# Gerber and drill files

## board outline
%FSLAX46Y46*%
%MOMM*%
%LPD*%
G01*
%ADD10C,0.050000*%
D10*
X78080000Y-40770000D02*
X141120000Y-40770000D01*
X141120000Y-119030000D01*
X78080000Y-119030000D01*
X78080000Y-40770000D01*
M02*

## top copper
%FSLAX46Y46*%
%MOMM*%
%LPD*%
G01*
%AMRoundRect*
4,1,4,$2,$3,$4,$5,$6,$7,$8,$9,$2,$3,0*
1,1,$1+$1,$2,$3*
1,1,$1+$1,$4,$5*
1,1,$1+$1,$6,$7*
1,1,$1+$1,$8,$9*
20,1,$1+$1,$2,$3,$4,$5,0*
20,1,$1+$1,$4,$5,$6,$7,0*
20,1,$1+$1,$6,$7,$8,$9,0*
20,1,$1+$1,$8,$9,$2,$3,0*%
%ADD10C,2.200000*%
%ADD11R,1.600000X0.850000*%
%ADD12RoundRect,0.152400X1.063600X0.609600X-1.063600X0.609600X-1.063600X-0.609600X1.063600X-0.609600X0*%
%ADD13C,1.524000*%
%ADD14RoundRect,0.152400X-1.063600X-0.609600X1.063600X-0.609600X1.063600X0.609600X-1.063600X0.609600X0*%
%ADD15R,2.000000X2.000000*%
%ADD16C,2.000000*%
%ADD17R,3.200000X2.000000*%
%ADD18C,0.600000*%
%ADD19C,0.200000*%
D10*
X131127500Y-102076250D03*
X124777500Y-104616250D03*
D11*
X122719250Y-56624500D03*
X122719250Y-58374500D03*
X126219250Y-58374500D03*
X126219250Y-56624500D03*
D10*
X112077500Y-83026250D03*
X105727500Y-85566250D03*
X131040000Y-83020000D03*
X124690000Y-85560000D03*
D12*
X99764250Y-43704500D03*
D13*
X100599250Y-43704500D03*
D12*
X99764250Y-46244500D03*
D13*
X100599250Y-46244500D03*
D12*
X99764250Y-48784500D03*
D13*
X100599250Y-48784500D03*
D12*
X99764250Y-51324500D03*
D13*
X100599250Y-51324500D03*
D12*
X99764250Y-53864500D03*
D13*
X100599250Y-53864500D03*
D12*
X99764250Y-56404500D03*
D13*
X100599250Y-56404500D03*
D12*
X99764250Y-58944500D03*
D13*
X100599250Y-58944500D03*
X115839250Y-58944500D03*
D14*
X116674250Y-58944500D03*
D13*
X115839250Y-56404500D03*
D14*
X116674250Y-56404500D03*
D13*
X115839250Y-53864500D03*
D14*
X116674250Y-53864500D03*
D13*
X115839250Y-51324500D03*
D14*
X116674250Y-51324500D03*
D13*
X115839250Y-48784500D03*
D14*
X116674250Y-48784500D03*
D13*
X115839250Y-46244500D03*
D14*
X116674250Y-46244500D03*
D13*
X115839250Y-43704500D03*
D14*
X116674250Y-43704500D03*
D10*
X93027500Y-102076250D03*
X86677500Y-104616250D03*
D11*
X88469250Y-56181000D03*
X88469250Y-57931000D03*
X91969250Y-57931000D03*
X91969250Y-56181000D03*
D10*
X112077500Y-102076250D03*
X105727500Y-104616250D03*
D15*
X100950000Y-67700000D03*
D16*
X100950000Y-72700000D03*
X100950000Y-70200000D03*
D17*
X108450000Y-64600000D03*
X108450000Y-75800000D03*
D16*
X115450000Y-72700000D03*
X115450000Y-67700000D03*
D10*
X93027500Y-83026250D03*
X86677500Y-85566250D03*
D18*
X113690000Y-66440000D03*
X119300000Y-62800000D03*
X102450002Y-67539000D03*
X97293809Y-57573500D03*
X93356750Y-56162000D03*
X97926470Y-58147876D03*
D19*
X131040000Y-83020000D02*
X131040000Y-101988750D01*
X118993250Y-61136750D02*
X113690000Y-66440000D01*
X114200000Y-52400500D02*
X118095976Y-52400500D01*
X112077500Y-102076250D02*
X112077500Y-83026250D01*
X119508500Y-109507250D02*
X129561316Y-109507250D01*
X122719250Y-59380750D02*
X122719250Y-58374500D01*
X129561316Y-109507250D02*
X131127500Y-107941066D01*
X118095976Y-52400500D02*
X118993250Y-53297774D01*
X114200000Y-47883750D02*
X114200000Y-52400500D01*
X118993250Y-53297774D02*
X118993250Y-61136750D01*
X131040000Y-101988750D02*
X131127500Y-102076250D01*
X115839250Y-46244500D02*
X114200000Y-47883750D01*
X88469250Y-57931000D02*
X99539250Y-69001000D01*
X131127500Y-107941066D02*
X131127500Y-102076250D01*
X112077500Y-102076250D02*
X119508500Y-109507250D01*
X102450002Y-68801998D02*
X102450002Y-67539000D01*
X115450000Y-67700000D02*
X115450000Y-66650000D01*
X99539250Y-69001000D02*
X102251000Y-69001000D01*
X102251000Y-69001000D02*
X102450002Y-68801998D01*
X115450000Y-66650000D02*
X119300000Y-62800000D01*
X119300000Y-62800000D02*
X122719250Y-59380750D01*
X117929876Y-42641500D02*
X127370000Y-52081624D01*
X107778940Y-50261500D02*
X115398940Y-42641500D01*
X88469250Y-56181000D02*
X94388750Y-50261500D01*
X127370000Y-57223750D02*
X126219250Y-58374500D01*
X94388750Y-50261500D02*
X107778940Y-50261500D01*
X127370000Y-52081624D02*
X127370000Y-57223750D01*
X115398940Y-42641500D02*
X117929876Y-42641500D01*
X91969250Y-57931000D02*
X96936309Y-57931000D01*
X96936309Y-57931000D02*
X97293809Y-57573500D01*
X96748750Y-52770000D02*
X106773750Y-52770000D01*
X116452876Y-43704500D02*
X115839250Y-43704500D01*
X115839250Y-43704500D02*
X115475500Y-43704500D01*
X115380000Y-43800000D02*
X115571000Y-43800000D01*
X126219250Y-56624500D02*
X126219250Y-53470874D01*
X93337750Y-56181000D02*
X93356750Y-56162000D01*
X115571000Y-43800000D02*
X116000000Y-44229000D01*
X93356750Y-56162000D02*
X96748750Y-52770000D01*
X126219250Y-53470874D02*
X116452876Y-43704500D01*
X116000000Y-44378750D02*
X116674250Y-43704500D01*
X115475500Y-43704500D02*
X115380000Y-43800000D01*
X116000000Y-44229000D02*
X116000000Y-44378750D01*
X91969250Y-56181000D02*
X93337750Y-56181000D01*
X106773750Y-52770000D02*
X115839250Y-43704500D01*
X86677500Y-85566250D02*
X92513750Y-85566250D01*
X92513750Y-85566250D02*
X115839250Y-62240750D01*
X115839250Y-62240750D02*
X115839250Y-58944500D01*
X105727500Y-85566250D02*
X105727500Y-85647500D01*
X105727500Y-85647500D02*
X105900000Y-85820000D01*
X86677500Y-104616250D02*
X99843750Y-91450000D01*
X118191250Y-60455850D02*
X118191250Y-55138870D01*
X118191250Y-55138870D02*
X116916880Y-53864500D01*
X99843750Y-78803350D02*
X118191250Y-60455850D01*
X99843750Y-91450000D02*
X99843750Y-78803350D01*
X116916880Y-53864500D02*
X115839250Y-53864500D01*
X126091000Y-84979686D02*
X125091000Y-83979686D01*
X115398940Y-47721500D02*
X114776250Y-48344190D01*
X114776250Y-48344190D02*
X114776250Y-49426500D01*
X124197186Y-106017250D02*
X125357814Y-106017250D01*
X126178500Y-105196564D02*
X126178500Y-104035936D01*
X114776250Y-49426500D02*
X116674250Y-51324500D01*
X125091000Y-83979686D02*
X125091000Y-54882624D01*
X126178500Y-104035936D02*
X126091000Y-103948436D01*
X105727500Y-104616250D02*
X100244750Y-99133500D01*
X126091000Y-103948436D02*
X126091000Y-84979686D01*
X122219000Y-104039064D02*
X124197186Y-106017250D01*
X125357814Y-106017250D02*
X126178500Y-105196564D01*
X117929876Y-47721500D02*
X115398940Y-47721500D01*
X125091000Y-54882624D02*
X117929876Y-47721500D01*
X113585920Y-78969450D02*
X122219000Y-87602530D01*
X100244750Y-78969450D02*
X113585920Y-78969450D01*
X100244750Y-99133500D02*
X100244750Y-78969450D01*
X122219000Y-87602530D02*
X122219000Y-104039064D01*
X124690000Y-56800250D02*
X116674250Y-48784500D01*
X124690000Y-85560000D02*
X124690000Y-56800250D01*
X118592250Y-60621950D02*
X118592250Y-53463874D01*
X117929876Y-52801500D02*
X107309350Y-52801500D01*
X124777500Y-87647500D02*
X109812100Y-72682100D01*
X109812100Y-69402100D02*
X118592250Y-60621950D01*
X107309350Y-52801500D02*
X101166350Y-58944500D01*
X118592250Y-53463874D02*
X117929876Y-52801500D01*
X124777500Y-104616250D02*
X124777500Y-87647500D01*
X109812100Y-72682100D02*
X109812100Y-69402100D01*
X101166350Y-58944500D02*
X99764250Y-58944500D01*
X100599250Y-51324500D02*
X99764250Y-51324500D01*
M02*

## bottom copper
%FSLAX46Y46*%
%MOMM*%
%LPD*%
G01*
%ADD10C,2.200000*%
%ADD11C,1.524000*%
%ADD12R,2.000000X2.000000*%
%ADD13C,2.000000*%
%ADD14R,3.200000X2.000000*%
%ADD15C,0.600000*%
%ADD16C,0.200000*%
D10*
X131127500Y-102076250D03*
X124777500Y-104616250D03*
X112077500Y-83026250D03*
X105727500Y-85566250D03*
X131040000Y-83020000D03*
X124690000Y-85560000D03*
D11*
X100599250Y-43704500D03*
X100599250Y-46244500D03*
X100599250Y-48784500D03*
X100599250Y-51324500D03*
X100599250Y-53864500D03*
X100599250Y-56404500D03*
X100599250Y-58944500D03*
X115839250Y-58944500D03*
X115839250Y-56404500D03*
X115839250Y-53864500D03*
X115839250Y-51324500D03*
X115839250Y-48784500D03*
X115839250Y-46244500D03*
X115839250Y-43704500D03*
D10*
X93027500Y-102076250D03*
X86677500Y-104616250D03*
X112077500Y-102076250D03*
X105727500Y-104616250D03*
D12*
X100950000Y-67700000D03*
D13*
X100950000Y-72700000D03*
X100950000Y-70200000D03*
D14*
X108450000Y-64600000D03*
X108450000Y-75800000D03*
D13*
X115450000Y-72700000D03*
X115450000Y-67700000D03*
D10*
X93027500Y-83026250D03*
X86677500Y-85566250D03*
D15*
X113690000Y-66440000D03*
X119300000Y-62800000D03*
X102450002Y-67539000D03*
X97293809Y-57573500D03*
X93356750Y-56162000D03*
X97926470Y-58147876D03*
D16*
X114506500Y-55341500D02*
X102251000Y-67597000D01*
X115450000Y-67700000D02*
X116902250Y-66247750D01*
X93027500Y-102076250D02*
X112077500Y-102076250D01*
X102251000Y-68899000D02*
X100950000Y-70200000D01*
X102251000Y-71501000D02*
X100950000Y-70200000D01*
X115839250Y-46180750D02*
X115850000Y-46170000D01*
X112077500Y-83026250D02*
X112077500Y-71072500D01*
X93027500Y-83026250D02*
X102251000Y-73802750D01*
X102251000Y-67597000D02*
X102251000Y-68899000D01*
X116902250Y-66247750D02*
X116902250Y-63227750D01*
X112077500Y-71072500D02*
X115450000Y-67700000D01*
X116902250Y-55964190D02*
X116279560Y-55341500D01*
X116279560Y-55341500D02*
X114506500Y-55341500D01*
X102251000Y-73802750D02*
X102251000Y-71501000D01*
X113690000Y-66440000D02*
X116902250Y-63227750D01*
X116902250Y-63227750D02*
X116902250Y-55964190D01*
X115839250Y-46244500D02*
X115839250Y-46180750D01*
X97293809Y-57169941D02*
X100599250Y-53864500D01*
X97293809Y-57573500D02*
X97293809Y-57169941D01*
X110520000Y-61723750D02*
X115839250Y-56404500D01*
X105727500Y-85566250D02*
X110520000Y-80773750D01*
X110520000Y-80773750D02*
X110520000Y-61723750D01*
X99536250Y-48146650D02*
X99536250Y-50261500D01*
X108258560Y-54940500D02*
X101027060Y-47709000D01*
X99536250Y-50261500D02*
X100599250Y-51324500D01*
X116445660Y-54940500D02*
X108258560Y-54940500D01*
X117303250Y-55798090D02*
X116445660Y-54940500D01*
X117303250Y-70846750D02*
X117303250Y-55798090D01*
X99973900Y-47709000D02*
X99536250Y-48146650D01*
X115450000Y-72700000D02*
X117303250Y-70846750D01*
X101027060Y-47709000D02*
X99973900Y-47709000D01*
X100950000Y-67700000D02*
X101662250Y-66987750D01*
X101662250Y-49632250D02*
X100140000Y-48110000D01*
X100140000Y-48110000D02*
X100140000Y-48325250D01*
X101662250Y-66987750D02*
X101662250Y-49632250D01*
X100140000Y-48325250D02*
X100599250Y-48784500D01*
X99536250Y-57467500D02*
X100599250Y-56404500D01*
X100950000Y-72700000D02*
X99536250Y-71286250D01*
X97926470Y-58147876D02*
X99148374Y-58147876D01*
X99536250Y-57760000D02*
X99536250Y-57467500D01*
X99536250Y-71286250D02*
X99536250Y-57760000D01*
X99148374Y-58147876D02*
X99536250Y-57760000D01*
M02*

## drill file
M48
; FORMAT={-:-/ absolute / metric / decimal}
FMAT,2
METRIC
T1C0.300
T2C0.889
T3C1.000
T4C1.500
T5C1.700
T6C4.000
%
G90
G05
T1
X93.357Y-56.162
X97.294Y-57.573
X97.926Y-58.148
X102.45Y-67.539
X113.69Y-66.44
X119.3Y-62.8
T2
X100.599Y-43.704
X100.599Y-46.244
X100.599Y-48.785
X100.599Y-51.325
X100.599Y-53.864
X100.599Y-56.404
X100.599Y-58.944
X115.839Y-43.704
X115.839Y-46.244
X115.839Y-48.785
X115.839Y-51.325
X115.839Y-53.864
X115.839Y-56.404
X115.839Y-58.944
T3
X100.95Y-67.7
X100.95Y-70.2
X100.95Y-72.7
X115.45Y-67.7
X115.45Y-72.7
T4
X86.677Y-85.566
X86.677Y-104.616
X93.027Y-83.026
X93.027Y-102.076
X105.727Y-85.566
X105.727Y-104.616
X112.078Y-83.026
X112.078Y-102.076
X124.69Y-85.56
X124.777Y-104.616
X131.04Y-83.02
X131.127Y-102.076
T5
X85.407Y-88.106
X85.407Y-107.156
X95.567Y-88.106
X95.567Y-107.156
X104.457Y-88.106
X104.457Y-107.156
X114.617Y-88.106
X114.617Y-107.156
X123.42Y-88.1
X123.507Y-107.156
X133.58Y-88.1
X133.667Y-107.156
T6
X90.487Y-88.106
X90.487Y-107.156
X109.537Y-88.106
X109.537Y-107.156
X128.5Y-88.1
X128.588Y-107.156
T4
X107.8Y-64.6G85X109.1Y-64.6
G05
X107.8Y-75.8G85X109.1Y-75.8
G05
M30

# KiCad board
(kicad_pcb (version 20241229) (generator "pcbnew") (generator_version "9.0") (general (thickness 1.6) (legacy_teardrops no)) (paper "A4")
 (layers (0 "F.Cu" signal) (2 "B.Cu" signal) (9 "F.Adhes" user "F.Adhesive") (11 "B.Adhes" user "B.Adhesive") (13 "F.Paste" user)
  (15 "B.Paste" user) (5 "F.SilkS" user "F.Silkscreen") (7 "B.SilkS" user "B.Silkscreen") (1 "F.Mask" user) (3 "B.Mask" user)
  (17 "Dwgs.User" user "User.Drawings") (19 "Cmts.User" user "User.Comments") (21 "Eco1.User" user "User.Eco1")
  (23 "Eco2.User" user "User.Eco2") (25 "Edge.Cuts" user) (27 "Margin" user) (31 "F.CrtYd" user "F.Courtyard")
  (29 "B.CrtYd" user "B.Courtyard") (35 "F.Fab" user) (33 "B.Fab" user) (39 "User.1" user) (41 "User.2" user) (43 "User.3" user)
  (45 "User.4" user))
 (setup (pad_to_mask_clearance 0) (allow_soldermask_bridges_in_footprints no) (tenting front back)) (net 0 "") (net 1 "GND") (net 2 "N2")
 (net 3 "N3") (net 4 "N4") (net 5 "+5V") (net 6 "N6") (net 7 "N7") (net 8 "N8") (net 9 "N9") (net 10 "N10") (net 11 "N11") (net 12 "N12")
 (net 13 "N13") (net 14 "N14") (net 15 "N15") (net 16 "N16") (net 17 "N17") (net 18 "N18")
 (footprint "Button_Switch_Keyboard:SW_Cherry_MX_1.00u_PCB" (layer "F.Cu") (at 131.1275 102.07625)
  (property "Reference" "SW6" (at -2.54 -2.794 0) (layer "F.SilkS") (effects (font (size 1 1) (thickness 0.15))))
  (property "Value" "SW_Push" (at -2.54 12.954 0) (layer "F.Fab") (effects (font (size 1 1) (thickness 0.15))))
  (pad "" np_thru_hole circle (at -7.62 5.08) (size 1.7 1.7) (drill 1.7) (layers "*.Cu" "*.Mask"))
  (pad "" np_thru_hole circle (at -2.54 5.08) (size 4 4) (drill 4) (layers "*.Cu" "*.Mask"))
  (pad "" np_thru_hole circle (at 2.54 5.08) (size 1.7 1.7) (drill 1.7) (layers "*.Cu" "*.Mask"))
  (pad "1" thru_hole circle (at 0 0) (size 2.2 2.2) (drill 1.5) (layers "*.Cu" "*.Mask") (remove_unused_layers no) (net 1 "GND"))
  (pad "2" thru_hole circle (at -6.35 2.54) (size 2.2 2.2) (drill 1.5) (layers "*.Cu" "*.Mask") (remove_unused_layers no) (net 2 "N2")))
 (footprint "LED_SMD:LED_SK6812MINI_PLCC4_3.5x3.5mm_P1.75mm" (layer "F.Cu") (at 124.46925 57.4995)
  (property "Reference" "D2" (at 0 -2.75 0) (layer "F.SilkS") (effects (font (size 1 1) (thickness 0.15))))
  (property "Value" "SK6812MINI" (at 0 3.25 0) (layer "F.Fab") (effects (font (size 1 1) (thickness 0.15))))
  (pad "1" smd rect (at -1.75 -0.875) (size 1.6 0.85) (layers "F.Cu" "F.Mask" "F.Paste") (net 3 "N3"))
  (pad "2" smd rect (at -1.75 0.875) (size 1.6 0.85) (layers "F.Cu" "F.Mask" "F.Paste") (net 1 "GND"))
  (pad "3" smd rect (at 1.75 0.875) (size 1.6 0.85) (layers "F.Cu" "F.Mask" "F.Paste") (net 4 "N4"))
  (pad "4" smd rect (at 1.75 -0.875) (size 1.6 0.85) (layers "F.Cu" "F.Mask" "F.Paste") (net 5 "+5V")))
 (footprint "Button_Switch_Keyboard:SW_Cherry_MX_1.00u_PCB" (layer "F.Cu") (at 112.0775 83.02625)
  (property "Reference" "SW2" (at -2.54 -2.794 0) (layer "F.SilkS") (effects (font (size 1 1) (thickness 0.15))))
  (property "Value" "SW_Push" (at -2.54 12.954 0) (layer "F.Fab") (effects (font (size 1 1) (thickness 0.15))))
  (pad "" np_thru_hole circle (at -7.62 5.08) (size 1.7 1.7) (drill 1.7) (layers "*.Cu" "*.Mask"))
  (pad "" np_thru_hole circle (at -2.54 5.08) (size 4 4) (drill 4) (layers "*.Cu" "*.Mask"))
  (pad "" np_thru_hole circle (at 2.54 5.08) (size 1.7 1.7) (drill 1.7) (layers "*.Cu" "*.Mask"))
  (pad "1" thru_hole circle (at 0 0) (size 2.2 2.2) (drill 1.5) (layers "*.Cu" "*.Mask") (remove_unused_layers no) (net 1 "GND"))
  (pad "2" thru_hole circle (at -6.35 2.54) (size 2.2 2.2) (drill 1.5) (layers "*.Cu" "*.Mask") (remove_unused_layers no) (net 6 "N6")))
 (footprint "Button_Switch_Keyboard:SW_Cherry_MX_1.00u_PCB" (layer "F.Cu") (at 131.04 83.02)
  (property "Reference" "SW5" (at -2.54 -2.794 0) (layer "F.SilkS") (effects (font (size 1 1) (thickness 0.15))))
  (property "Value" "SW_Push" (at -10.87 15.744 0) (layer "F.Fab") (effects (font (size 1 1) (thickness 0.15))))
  (pad "" np_thru_hole circle (at -7.62 5.08) (size 1.7 1.7) (drill 1.7) (layers "*.Cu" "*.Mask"))
  (pad "" np_thru_hole circle (at -2.54 5.08) (size 4 4) (drill 4) (layers "*.Cu" "*.Mask"))
  (pad "" np_thru_hole circle (at 2.54 5.08) (size 1.7 1.7) (drill 1.7) (layers "*.Cu" "*.Mask"))
  (pad "1" thru_hole circle (at 0 0) (size 2.2 2.2) (drill 1.5) (layers "*.Cu" "*.Mask") (remove_unused_layers no) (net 1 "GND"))
  (pad "2" thru_hole circle (at -6.35 2.54) (size 2.2 2.2) (drill 1.5) (layers "*.Cu" "*.Mask") (remove_unused_layers no) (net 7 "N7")))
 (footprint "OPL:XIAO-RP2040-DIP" (layer "F.Cu") (at 108.21925 51.3245)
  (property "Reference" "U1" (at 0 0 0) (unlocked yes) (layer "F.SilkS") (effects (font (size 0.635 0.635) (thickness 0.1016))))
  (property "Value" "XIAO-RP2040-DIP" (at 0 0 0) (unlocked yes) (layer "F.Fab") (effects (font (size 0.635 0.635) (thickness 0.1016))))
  (pad "1" smd roundrect (at -8.455 -7.62 180) (size 2.432 1.524) (layers "F.Cu" "F.Mask") (roundrect_rratio 0.1) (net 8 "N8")
   (thermal_bridge_angle 45))
  (pad "1" thru_hole circle (at -7.62 -7.62 180) (size 1.524 1.524) (drill 0.889) (layers "*.Cu" "*.Mask") (remove_unused_layers no)
   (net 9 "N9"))
  (pad "2" smd roundrect (at -8.455 -5.08 180) (size 2.432 1.524) (layers "F.Cu" "F.Mask") (roundrect_rratio 0.1) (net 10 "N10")
   (thermal_bridge_angle 45))
  (pad "2" thru_hole circle (at -7.62 -5.08 180) (size 1.524 1.524) (drill 0.889) (layers "*.Cu" "*.Mask") (remove_unused_layers no)
   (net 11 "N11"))
  (pad "3" smd roundrect (at -8.455 -2.54 180) (size 2.432 1.524) (layers "F.Cu" "F.Mask") (roundrect_rratio 0.1) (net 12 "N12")
   (thermal_bridge_angle 45))
  (pad "3" thru_hole circle (at -7.62 -2.54 180) (size 1.524 1.524) (drill 0.889) (layers "*.Cu" "*.Mask") (remove_unused_layers no)
   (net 12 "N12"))
  (pad "4" smd roundrect (at -8.455 0 180) (size 2.432 1.524) (layers "F.Cu" "F.Mask") (roundrect_rratio 0.1) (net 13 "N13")
   (thermal_bridge_angle 45))
  (pad "4" thru_hole circle (at -7.62 0 180) (size 1.524 1.524) (drill 0.889) (layers "*.Cu" "*.Mask") (remove_unused_layers no)
   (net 13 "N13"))
  (pad "5" smd roundrect (at -8.455 2.54 180) (size 2.432 1.524) (layers "F.Cu" "F.Mask") (roundrect_rratio 0.1) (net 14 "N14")
   (thermal_bridge_angle 45))
  (pad "5" thru_hole circle (at -7.62 2.54 180) (size 1.524 1.524) (drill 0.889) (layers "*.Cu" "*.Mask") (remove_unused_layers no)
   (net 14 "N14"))
  (pad "6" smd roundrect (at -8.455 5.08 180) (size 2.432 1.524) (layers "F.Cu" "F.Mask") (roundrect_rratio 0.1) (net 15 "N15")
   (thermal_bridge_angle 45))
  (pad "6" thru_hole circle (at -7.62 5.08 180) (size 1.524 1.524) (drill 0.889) (layers "*.Cu" "*.Mask") (remove_unused_layers no)
   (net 15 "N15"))
  (pad "7" smd roundrect (at -8.455 7.62 180) (size 2.432 1.524) (layers "F.Cu" "F.Mask") (roundrect_rratio 0.1) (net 2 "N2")
   (thermal_bridge_angle 45))
  (pad "7" thru_hole circle (at -7.62 7.62 180) (size 1.524 1.524) (drill 0.889) (layers "*.Cu" "*.Mask") (remove_unused_layers no)
   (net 2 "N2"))
  (pad "8" thru_hole circle (at 7.62 7.62) (size 1.524 1.524) (drill 0.889) (layers "*.Cu" "*.Mask") (remove_unused_layers no)
   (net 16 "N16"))
  (pad "8" smd roundrect (at 8.455 7.62) (size 2.432 1.524) (layers "F.Cu" "F.Mask") (roundrect_rratio 0.1) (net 16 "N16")
   (thermal_bridge_angle 45))
  (pad "9" thru_hole circle (at 7.62 5.08) (size 1.524 1.524) (drill 0.889) (layers "*.Cu" "*.Mask") (remove_unused_layers no) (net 6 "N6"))
  (pad "9" smd roundrect (at 8.455 5.08) (size 2.432 1.524) (layers "F.Cu" "F.Mask") (roundrect_rratio 0.1) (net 6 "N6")
   (thermal_bridge_angle 45))
  (pad "10" thru_hole circle (at 7.62 2.54) (size 1.524 1.524) (drill 0.889) (layers "*.Cu" "*.Mask") (remove_unused_layers no)
   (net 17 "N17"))
  (pad "10" smd roundrect (at 8.455 2.54) (size 2.432 1.524) (layers "F.Cu" "F.Mask") (roundrect_rratio 0.1) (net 17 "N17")
   (thermal_bridge_angle 45))
  (pad "11" thru_hole circle (at 7.62 0) (size 1.524 1.524) (drill 0.889) (layers "*.Cu" "*.Mask") (remove_unused_layers no) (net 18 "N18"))
  (pad "11" smd roundrect (at 8.455 0) (size 2.432 1.524) (layers "F.Cu" "F.Mask") (roundrect_rratio 0.1) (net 18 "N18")
   (thermal_bridge_angle 45))
  (pad "12" thru_hole circle (at 7.62 -2.54) (size 1.524 1.524) (drill 0.889) (layers "*.Cu" "*.Mask") (remove_unused_layers no)
   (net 7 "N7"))
  (pad "12" smd roundrect (at 8.455 -2.54) (size 2.432 1.524) (layers "F.Cu" "F.Mask") (roundrect_rratio 0.1) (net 7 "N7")
   (thermal_bridge_angle 45))
  (pad "13" thru_hole circle (at 7.62 -5.08) (size 1.524 1.524) (drill 0.889) (layers "*.Cu" "*.Mask") (remove_unused_layers no)
   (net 1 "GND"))
  (pad "13" smd roundrect (at 8.455 -5.08) (size 2.432 1.524) (layers "F.Cu" "F.Mask") (roundrect_rratio 0.1) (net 1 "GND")
   (thermal_bridge_angle 45))
  (pad "14" thru_hole circle (at 7.62 -7.62) (size 1.524 1.524) (drill 0.889) (layers "*.Cu" "*.Mask") (remove_unused_layers no)
   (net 5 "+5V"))
  (pad "14" smd roundrect (at 8.455 -7.62) (size 2.432 1.524) (layers "F.Cu" "F.Mask") (roundrect_rratio 0.1) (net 5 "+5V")
   (thermal_bridge_angle 45)))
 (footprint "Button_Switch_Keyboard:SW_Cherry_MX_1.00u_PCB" (layer "F.Cu") (at 93.0275 102.07625)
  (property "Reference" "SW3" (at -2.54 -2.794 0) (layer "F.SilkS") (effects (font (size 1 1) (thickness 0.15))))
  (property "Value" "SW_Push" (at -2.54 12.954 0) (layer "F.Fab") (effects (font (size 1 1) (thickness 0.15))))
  (pad "" np_thru_hole circle (at -7.62 5.08) (size 1.7 1.7) (drill 1.7) (layers "*.Cu" "*.Mask"))
  (pad "" np_thru_hole circle (at -2.54 5.08) (size 4 4) (drill 4) (layers "*.Cu" "*.Mask"))
  (pad "" np_thru_hole circle (at 2.54 5.08) (size 1.7 1.7) (drill 1.7) (layers "*.Cu" "*.Mask"))
  (pad "1" thru_hole circle (at 0 0) (size 2.2 2.2) (drill 1.5) (layers "*.Cu" "*.Mask") (remove_unused_layers no) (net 1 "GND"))
  (pad "2" thru_hole circle (at -6.35 2.54) (size 2.2 2.2) (drill 1.5) (layers "*.Cu" "*.Mask") (remove_unused_layers no) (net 17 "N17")))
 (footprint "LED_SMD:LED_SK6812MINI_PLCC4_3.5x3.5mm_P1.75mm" (layer "F.Cu") (at 90.21925 57.056)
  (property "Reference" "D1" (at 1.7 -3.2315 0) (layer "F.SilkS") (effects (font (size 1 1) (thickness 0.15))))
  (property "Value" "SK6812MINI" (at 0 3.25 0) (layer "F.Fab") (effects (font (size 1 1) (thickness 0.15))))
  (pad "1" smd rect (at -1.75 -0.875) (size 1.6 0.85) (layers "F.Cu" "F.Mask" "F.Paste") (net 4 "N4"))
  (pad "2" smd rect (at -1.75 0.875) (size 1.6 0.85) (layers "F.Cu" "F.Mask" "F.Paste") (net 1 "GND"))
  (pad "3" smd rect (at 1.75 0.875) (size 1.6 0.85) (layers "F.Cu" "F.Mask" "F.Paste") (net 14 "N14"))
  (pad "4" smd rect (at 1.75 -0.875) (size 1.6 0.85) (layers "F.Cu" "F.Mask" "F.Paste") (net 5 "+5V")))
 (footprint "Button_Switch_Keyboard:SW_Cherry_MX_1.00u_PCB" (layer "F.Cu") (at 112.0775 102.07625)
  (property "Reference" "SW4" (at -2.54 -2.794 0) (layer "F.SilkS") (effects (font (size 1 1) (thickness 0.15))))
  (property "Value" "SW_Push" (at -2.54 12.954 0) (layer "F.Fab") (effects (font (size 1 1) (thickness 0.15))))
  (pad "" np_thru_hole circle (at -7.62 5.08) (size 1.7 1.7) (drill 1.7) (layers "*.Cu" "*.Mask"))
  (pad "" np_thru_hole circle (at -2.54 5.08) (size 4 4) (drill 4) (layers "*.Cu" "*.Mask"))
  (pad "" np_thru_hole circle (at 2.54 5.08) (size 1.7 1.7) (drill 1.7) (layers "*.Cu" "*.Mask"))
  (pad "1" thru_hole circle (at 0 0) (size 2.2 2.2) (drill 1.5) (layers "*.Cu" "*.Mask") (remove_unused_layers no) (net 1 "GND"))
  (pad "2" thru_hole circle (at -6.35 2.54) (size 2.2 2.2) (drill 1.5) (layers "*.Cu" "*.Mask") (remove_unused_layers no) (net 18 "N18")))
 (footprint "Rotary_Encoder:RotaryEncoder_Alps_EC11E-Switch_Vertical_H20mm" (layer "F.Cu") (at 100.95 67.7)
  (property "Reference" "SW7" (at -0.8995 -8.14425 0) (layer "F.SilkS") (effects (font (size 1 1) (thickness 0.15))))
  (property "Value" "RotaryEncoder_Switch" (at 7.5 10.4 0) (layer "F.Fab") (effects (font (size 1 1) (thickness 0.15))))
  (pad "A" thru_hole rect (at 0 0) (size 2 2) (drill 1) (layers "*.Cu" "*.Mask") (remove_unused_layers no) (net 12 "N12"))
  (pad "B" thru_hole circle (at 0 5) (size 2 2) (drill 1) (layers "*.Cu" "*.Mask") (remove_unused_layers no) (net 15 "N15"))
  (pad "C" thru_hole circle (at 0 2.5) (size 2 2) (drill 1) (layers "*.Cu" "*.Mask") (remove_unused_layers no) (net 1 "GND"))
  (pad "MP" thru_hole rect (at 7.5 -3.1) (size 3.2 2) (drill oval 2.8 1.5) (layers "*.Cu" "*.Mask") (remove_unused_layers no))
  (pad "MP" thru_hole rect (at 7.5 8.1) (size 3.2 2) (drill oval 2.8 1.5) (layers "*.Cu" "*.Mask") (remove_unused_layers no))
  (pad "S1" thru_hole circle (at 14.5 5) (size 2 2) (drill 1) (layers "*.Cu" "*.Mask") (remove_unused_layers no) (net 13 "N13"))
  (pad "S2" thru_hole circle (at 14.5 0) (size 2 2) (drill 1) (layers "*.Cu" "*.Mask") (remove_unused_layers no) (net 1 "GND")))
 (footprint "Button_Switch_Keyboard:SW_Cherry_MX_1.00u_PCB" (layer "F.Cu") (at 93.0275 83.02625)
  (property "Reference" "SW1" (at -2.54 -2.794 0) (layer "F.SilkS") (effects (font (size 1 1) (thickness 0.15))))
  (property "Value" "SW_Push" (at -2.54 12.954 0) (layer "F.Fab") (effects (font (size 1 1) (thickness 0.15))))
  (pad "" np_thru_hole circle (at -7.62 5.08) (size 1.7 1.7) (drill 1.7) (layers "*.Cu" "*.Mask"))
  (pad "" np_thru_hole circle (at -2.54 5.08) (size 4 4) (drill 4) (layers "*.Cu" "*.Mask"))
  (pad "" np_thru_hole circle (at 2.54 5.08) (size 1.7 1.7) (drill 1.7) (layers "*.Cu" "*.Mask"))
  (pad "1" thru_hole circle (at 0 0) (size 2.2 2.2) (drill 1.5) (layers "*.Cu" "*.Mask") (remove_unused_layers no) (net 1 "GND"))
  (pad "2" thru_hole circle (at -6.35 2.54) (size 2.2 2.2) (drill 1.5) (layers "*.Cu" "*.Mask") (remove_unused_layers no) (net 16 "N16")))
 (gr_rect (start 78.08 40.77) (end 141.12 119.03) (stroke (width 0.05) (type default)) (fill no) (layer "Edge.Cuts"))
 (segment (start 131.04 83.02) (end 131.04 101.98875) (width 0.2) (layer "F.Cu") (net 1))
 (segment (start 118.99325 61.13675) (end 113.69 66.44) (width 0.2) (layer "F.Cu") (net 1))
 (segment (start 114.2 52.4005) (end 118.095976 52.4005) (width 0.2) (layer "F.Cu") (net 1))
 (segment (start 112.0775 102.07625) (end 112.0775 83.02625) (width 0.2) (layer "F.Cu") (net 1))
 (segment (start 119.5085 109.50725) (end 129.561316 109.50725) (width 0.2) (layer "F.Cu") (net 1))
 (segment (start 122.71925 59.38075) (end 122.71925 58.3745) (width 0.2) (layer "F.Cu") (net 1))
 (segment (start 129.561316 109.50725) (end 131.1275 107.941066) (width 0.2) (layer "F.Cu") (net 1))
 (segment (start 118.095976 52.4005) (end 118.99325 53.297774) (width 0.2) (layer "F.Cu") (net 1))
 (segment (start 114.2 47.88375) (end 114.2 52.4005) (width 0.2) (layer "F.Cu") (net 1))
 (segment (start 118.99325 53.297774) (end 118.99325 61.13675) (width 0.2) (layer "F.Cu") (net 1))
 (segment (start 131.04 101.98875) (end 131.1275 102.07625) (width 0.2) (layer "F.Cu") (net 1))
 (segment (start 115.83925 46.2445) (end 114.2 47.88375) (width 0.2) (layer "F.Cu") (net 1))
 (segment (start 88.46925 57.931) (end 99.53925 69.001) (width 0.2) (layer "F.Cu") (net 1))
 (segment (start 131.1275 107.941066) (end 131.1275 102.07625) (width 0.2) (layer "F.Cu") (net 1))
 (segment (start 112.0775 102.07625) (end 119.5085 109.50725) (width 0.2) (layer "F.Cu") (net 1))
 (segment (start 102.450002 68.801998) (end 102.450002 67.539) (width 0.2) (layer "F.Cu") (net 1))
 (segment (start 115.45 67.7) (end 115.45 66.65) (width 0.2) (layer "F.Cu") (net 1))
 (segment (start 99.53925 69.001) (end 102.251 69.001) (width 0.2) (layer "F.Cu") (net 1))
 (segment (start 102.251 69.001) (end 102.450002 68.801998) (width 0.2) (layer "F.Cu") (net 1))
 (segment (start 115.45 66.65) (end 119.3 62.8) (width 0.2) (layer "F.Cu") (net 1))
 (segment (start 119.3 62.8) (end 122.71925 59.38075) (width 0.2) (layer "F.Cu") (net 1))
 (via (at 113.69 66.44) (size 0.6) (drill 0.3) (layers "F.Cu" "B.Cu") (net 1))
 (via (at 119.3 62.8) (size 0.6) (drill 0.3) (layers "F.Cu" "B.Cu") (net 1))
 (via (at 102.450002 67.539) (size 0.6) (drill 0.3) (layers "F.Cu" "B.Cu") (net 1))
 (segment (start 114.5065 55.3415) (end 102.251 67.597) (width 0.2) (layer "B.Cu") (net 1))
 (segment (start 115.45 67.7) (end 116.90225 66.24775) (width 0.2) (layer "B.Cu") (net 1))
 (segment (start 93.0275 102.07625) (end 112.0775 102.07625) (width 0.2) (layer "B.Cu") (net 1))
 (segment (start 102.251 68.899) (end 100.95 70.2) (width 0.2) (layer "B.Cu") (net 1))
 (segment (start 102.251 71.501) (end 100.95 70.2) (width 0.2) (layer "B.Cu") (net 1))
 (segment (start 115.83925 46.18075) (end 115.85 46.17) (width 0.2) (layer "B.Cu") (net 1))
 (segment (start 112.0775 83.02625) (end 112.0775 71.0725) (width 0.2) (layer "B.Cu") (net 1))
 (segment (start 93.0275 83.02625) (end 102.251 73.80275) (width 0.2) (layer "B.Cu") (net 1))
 (segment (start 102.251 67.597) (end 102.251 68.899) (width 0.2) (layer "B.Cu") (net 1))
 (segment (start 116.90225 66.24775) (end 116.90225 63.22775) (width 0.2) (layer "B.Cu") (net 1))
 (segment (start 112.0775 71.0725) (end 115.45 67.7) (width 0.2) (layer "B.Cu") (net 1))
 (segment (start 116.90225 55.96419) (end 116.27956 55.3415) (width 0.2) (layer "B.Cu") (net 1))
 (segment (start 116.27956 55.3415) (end 114.5065 55.3415) (width 0.2) (layer "B.Cu") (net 1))
 (segment (start 102.251 73.80275) (end 102.251 71.501) (width 0.2) (layer "B.Cu") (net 1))
 (segment (start 113.69 66.44) (end 116.90225 63.22775) (width 0.2) (layer "B.Cu") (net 1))
 (segment (start 116.90225 63.22775) (end 116.90225 55.96419) (width 0.2) (layer "B.Cu") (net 1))
 (segment (start 115.83925 46.2445) (end 115.83925 46.18075) (width 0.2) (layer "B.Cu") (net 1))
 (segment (start 117.929876 42.6415) (end 127.37 52.081624) (width 0.2) (layer "F.Cu") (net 4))
 (segment (start 107.77894 50.2615) (end 115.39894 42.6415) (width 0.2) (layer "F.Cu") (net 4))
 (segment (start 88.46925 56.181) (end 94.38875 50.2615) (width 0.2) (layer "F.Cu") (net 4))
 (segment (start 127.37 57.22375) (end 126.21925 58.3745) (width 0.2) (layer "F.Cu") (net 4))
 (segment (start 94.38875 50.2615) (end 107.77894 50.2615) (width 0.2) (layer "F.Cu") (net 4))
 (segment (start 127.37 52.081624) (end 127.37 57.22375) (width 0.2) (layer "F.Cu") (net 4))
 (segment (start 115.39894 42.6415) (end 117.929876 42.6415) (width 0.2) (layer "F.Cu") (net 4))
 (segment (start 91.96925 57.931) (end 96.936309 57.931) (width 0.2) (layer "F.Cu") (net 14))
 (segment (start 96.936309 57.931) (end 97.293809 57.5735) (width 0.2) (layer "F.Cu") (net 14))
 (via (at 97.293809 57.5735) (size 0.6) (drill 0.3) (layers "F.Cu" "B.Cu") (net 14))
 (segment (start 97.293809 57.169941) (end 100.59925 53.8645) (width 0.2) (layer "B.Cu") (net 14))
 (segment (start 97.293809 57.5735) (end 97.293809 57.169941) (width 0.2) (layer "B.Cu") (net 14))
 (segment (start 96.74875 52.77) (end 106.77375 52.77) (width 0.2) (layer "F.Cu") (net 5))
 (segment (start 116.452876 43.7045) (end 115.83925 43.7045) (width 0.2) (layer "F.Cu") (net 5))
 (segment (start 115.83925 43.7045) (end 115.4755 43.7045) (width 0.2) (layer "F.Cu") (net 5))
 (segment (start 115.38 43.8) (end 115.571 43.8) (width 0.2) (layer "F.Cu") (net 5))
 (segment (start 126.21925 56.6245) (end 126.21925 53.470874) (width 0.2) (layer "F.Cu") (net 5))
 (segment (start 93.33775 56.181) (end 93.35675 56.162) (width 0.2) (layer "F.Cu") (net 5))
 (segment (start 115.571 43.8) (end 116 44.229) (width 0.2) (layer "F.Cu") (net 5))
 (segment (start 93.35675 56.162) (end 96.74875 52.77) (width 0.2) (layer "F.Cu") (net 5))
 (segment (start 126.21925 53.470874) (end 116.452876 43.7045) (width 0.2) (layer "F.Cu") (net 5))
 (segment (start 116 44.37875) (end 116.67425 43.7045) (width 0.2) (layer "F.Cu") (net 5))
 (segment (start 115.4755 43.7045) (end 115.38 43.8) (width 0.2) (layer "F.Cu") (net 5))
 (segment (start 116 44.229) (end 116 44.37875) (width 0.2) (layer "F.Cu") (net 5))
 (segment (start 91.96925 56.181) (end 93.33775 56.181) (width 0.2) (layer "F.Cu") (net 5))
 (segment (start 106.77375 52.77) (end 115.83925 43.7045) (width 0.2) (layer "F.Cu") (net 5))
 (via (at 93.35675 56.162) (size 0.6) (drill 0.3) (layers "F.Cu" "B.Cu") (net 5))
 (segment (start 86.6775 85.56625) (end 92.51375 85.56625) (width 0.2) (layer "F.Cu") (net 16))
 (segment (start 92.51375 85.56625) (end 115.83925 62.24075) (width 0.2) (layer "F.Cu") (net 16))
 (segment (start 115.83925 62.24075) (end 115.83925 58.9445) (width 0.2) (layer "F.Cu") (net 16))
 (segment (start 105.7275 85.56625) (end 105.7275 85.6475) (width 0.2) (layer "F.Cu") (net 6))
 (segment (start 105.7275 85.6475) (end 105.9 85.82) (width 0.2) (layer "F.Cu") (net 6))
 (segment (start 110.52 61.72375) (end 115.83925 56.4045) (width 0.2) (layer "B.Cu") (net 6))
 (segment (start 105.7275 85.56625) (end 110.52 80.77375) (width 0.2) (layer "B.Cu") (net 6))
 (segment (start 110.52 80.77375) (end 110.52 61.72375) (width 0.2) (layer "B.Cu") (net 6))
 (segment (start 86.6775 104.61625) (end 99.84375 91.45) (width 0.2) (layer "F.Cu") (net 17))
 (segment (start 118.19125 60.45585) (end 118.19125 55.13887) (width 0.2) (layer "F.Cu") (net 17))
 (segment (start 118.19125 55.13887) (end 116.91688 53.8645) (width 0.2) (layer "F.Cu") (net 17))
 (segment (start 99.84375 78.80335) (end 118.19125 60.45585) (width 0.2) (layer "F.Cu") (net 17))
 (segment (start 99.84375 91.45) (end 99.84375 78.80335) (width 0.2) (layer "F.Cu") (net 17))
 (segment (start 116.91688 53.8645) (end 115.83925 53.8645) (width 0.2) (layer "F.Cu") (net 17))
 (segment (start 126.091 84.979686) (end 125.091 83.979686) (width 0.2) (layer "F.Cu") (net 18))
 (segment (start 115.39894 47.7215) (end 114.77625 48.34419) (width 0.2) (layer "F.Cu") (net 18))
 (segment (start 114.77625 48.34419) (end 114.77625 49.4265) (width 0.2) (layer "F.Cu") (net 18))
 (segment (start 124.197186 106.01725) (end 125.357814 106.01725) (width 0.2) (layer "F.Cu") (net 18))
 (segment (start 126.1785 105.196564) (end 126.1785 104.035936) (width 0.2) (layer "F.Cu") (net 18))
 (segment (start 114.77625 49.4265) (end 116.67425 51.3245) (width 0.2) (layer "F.Cu") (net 18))
 (segment (start 125.091 83.979686) (end 125.091 54.882624) (width 0.2) (layer "F.Cu") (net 18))
 (segment (start 126.1785 104.035936) (end 126.091 103.948436) (width 0.2) (layer "F.Cu") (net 18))
 (segment (start 105.7275 104.61625) (end 100.24475 99.1335) (width 0.2) (layer "F.Cu") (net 18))
 (segment (start 126.091 103.948436) (end 126.091 84.979686) (width 0.2) (layer "F.Cu") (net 18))
 (segment (start 122.219 104.039064) (end 124.197186 106.01725) (width 0.2) (layer "F.Cu") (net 18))
 (segment (start 125.357814 106.01725) (end 126.1785 105.196564) (width 0.2) (layer "F.Cu") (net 18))
 (segment (start 117.929876 47.7215) (end 115.39894 47.7215) (width 0.2) (layer "F.Cu") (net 18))
 (segment (start 125.091 54.882624) (end 117.929876 47.7215) (width 0.2) (layer "F.Cu") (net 18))
 (segment (start 113.58592 78.96945) (end 122.219 87.60253) (width 0.2) (layer "F.Cu") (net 18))
 (segment (start 100.24475 78.96945) (end 113.58592 78.96945) (width 0.2) (layer "F.Cu") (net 18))
 (segment (start 100.24475 99.1335) (end 100.24475 78.96945) (width 0.2) (layer "F.Cu") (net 18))
 (segment (start 122.219 87.60253) (end 122.219 104.039064) (width 0.2) (layer "F.Cu") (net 18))
 (segment (start 124.69 56.80025) (end 116.67425 48.7845) (width 0.2) (layer "F.Cu") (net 7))
 (segment (start 124.69 85.56) (end 124.69 56.80025) (width 0.2) (layer "F.Cu") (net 7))
 (segment (start 118.59225 60.62195) (end 118.59225 53.463874) (width 0.2) (layer "F.Cu") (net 2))
 (segment (start 117.929876 52.8015) (end 107.30935 52.8015) (width 0.2) (layer "F.Cu") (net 2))
 (segment (start 124.7775 87.6475) (end 109.8121 72.6821) (width 0.2) (layer "F.Cu") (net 2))
 (segment (start 109.8121 69.4021) (end 118.59225 60.62195) (width 0.2) (layer "F.Cu") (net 2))
 (segment (start 107.30935 52.8015) (end 101.16635 58.9445) (width 0.2) (layer "F.Cu") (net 2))
 (segment (start 118.59225 53.463874) (end 117.929876 52.8015) (width 0.2) (layer "F.Cu") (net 2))
 (segment (start 124.7775 104.61625) (end 124.7775 87.6475) (width 0.2) (layer "F.Cu") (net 2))
 (segment (start 109.8121 72.6821) (end 109.8121 69.4021) (width 0.2) (layer "F.Cu") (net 2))
 (segment (start 101.16635 58.9445) (end 99.76425 58.9445) (width 0.2) (layer "F.Cu") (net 2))
 (segment (start 100.59925 51.3245) (end 99.76425 51.3245) (width 0.2) (layer "F.Cu") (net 13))
 (segment (start 99.53625 48.14665) (end 99.53625 50.2615) (width 0.2) (layer "B.Cu") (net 13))
 (segment (start 108.25856 54.9405) (end 101.02706 47.709) (width 0.2) (layer "B.Cu") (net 13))
 (segment (start 99.53625 50.2615) (end 100.59925 51.3245) (width 0.2) (layer "B.Cu") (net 13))
 (segment (start 116.44566 54.9405) (end 108.25856 54.9405) (width 0.2) (layer "B.Cu") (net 13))
 (segment (start 117.30325 55.79809) (end 116.44566 54.9405) (width 0.2) (layer "B.Cu") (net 13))
 (segment (start 117.30325 70.84675) (end 117.30325 55.79809) (width 0.2) (layer "B.Cu") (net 13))
 (segment (start 99.9739 47.709) (end 99.53625 48.14665) (width 0.2) (layer "B.Cu") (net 13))
 (segment (start 115.45 72.7) (end 117.30325 70.84675) (width 0.2) (layer "B.Cu") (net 13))
 (segment (start 101.02706 47.709) (end 99.9739 47.709) (width 0.2) (layer "B.Cu") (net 13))
 (segment (start 100.95 67.7) (end 101.66225 66.98775) (width 0.2) (layer "B.Cu") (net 12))
 (segment (start 101.66225 49.63225) (end 100.14 48.11) (width 0.2) (layer "B.Cu") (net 12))
 (segment (start 100.14 48.11) (end 100.14 48.32525) (width 0.2) (layer "B.Cu") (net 12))
 (segment (start 101.66225 66.98775) (end 101.66225 49.63225) (width 0.2) (layer "B.Cu") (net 12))
 (segment (start 100.14 48.32525) (end 100.59925 48.7845) (width 0.2) (layer "B.Cu") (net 12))
 (via (at 97.92647 58.147876) (size 0.6) (drill 0.3) (layers "F.Cu" "B.Cu") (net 15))
 (segment (start 99.53625 57.4675) (end 100.59925 56.4045) (width 0.2) (layer "B.Cu") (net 15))
 (segment (start 100.95 72.7) (end 99.53625 71.28625) (width 0.2) (layer "B.Cu") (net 15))
 (segment (start 97.92647 58.147876) (end 99.148374 58.147876) (width 0.2) (layer "B.Cu") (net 15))
 (segment (start 99.53625 57.76) (end 99.53625 57.4675) (width 0.2) (layer "B.Cu") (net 15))
 (segment (start 99.53625 71.28625) (end 99.53625 57.76) (width 0.2) (layer "B.Cu") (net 15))
 (segment (start 99.148374 58.147876) (end 99.53625 57.76) (width 0.2) (layer "B.Cu") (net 15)))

